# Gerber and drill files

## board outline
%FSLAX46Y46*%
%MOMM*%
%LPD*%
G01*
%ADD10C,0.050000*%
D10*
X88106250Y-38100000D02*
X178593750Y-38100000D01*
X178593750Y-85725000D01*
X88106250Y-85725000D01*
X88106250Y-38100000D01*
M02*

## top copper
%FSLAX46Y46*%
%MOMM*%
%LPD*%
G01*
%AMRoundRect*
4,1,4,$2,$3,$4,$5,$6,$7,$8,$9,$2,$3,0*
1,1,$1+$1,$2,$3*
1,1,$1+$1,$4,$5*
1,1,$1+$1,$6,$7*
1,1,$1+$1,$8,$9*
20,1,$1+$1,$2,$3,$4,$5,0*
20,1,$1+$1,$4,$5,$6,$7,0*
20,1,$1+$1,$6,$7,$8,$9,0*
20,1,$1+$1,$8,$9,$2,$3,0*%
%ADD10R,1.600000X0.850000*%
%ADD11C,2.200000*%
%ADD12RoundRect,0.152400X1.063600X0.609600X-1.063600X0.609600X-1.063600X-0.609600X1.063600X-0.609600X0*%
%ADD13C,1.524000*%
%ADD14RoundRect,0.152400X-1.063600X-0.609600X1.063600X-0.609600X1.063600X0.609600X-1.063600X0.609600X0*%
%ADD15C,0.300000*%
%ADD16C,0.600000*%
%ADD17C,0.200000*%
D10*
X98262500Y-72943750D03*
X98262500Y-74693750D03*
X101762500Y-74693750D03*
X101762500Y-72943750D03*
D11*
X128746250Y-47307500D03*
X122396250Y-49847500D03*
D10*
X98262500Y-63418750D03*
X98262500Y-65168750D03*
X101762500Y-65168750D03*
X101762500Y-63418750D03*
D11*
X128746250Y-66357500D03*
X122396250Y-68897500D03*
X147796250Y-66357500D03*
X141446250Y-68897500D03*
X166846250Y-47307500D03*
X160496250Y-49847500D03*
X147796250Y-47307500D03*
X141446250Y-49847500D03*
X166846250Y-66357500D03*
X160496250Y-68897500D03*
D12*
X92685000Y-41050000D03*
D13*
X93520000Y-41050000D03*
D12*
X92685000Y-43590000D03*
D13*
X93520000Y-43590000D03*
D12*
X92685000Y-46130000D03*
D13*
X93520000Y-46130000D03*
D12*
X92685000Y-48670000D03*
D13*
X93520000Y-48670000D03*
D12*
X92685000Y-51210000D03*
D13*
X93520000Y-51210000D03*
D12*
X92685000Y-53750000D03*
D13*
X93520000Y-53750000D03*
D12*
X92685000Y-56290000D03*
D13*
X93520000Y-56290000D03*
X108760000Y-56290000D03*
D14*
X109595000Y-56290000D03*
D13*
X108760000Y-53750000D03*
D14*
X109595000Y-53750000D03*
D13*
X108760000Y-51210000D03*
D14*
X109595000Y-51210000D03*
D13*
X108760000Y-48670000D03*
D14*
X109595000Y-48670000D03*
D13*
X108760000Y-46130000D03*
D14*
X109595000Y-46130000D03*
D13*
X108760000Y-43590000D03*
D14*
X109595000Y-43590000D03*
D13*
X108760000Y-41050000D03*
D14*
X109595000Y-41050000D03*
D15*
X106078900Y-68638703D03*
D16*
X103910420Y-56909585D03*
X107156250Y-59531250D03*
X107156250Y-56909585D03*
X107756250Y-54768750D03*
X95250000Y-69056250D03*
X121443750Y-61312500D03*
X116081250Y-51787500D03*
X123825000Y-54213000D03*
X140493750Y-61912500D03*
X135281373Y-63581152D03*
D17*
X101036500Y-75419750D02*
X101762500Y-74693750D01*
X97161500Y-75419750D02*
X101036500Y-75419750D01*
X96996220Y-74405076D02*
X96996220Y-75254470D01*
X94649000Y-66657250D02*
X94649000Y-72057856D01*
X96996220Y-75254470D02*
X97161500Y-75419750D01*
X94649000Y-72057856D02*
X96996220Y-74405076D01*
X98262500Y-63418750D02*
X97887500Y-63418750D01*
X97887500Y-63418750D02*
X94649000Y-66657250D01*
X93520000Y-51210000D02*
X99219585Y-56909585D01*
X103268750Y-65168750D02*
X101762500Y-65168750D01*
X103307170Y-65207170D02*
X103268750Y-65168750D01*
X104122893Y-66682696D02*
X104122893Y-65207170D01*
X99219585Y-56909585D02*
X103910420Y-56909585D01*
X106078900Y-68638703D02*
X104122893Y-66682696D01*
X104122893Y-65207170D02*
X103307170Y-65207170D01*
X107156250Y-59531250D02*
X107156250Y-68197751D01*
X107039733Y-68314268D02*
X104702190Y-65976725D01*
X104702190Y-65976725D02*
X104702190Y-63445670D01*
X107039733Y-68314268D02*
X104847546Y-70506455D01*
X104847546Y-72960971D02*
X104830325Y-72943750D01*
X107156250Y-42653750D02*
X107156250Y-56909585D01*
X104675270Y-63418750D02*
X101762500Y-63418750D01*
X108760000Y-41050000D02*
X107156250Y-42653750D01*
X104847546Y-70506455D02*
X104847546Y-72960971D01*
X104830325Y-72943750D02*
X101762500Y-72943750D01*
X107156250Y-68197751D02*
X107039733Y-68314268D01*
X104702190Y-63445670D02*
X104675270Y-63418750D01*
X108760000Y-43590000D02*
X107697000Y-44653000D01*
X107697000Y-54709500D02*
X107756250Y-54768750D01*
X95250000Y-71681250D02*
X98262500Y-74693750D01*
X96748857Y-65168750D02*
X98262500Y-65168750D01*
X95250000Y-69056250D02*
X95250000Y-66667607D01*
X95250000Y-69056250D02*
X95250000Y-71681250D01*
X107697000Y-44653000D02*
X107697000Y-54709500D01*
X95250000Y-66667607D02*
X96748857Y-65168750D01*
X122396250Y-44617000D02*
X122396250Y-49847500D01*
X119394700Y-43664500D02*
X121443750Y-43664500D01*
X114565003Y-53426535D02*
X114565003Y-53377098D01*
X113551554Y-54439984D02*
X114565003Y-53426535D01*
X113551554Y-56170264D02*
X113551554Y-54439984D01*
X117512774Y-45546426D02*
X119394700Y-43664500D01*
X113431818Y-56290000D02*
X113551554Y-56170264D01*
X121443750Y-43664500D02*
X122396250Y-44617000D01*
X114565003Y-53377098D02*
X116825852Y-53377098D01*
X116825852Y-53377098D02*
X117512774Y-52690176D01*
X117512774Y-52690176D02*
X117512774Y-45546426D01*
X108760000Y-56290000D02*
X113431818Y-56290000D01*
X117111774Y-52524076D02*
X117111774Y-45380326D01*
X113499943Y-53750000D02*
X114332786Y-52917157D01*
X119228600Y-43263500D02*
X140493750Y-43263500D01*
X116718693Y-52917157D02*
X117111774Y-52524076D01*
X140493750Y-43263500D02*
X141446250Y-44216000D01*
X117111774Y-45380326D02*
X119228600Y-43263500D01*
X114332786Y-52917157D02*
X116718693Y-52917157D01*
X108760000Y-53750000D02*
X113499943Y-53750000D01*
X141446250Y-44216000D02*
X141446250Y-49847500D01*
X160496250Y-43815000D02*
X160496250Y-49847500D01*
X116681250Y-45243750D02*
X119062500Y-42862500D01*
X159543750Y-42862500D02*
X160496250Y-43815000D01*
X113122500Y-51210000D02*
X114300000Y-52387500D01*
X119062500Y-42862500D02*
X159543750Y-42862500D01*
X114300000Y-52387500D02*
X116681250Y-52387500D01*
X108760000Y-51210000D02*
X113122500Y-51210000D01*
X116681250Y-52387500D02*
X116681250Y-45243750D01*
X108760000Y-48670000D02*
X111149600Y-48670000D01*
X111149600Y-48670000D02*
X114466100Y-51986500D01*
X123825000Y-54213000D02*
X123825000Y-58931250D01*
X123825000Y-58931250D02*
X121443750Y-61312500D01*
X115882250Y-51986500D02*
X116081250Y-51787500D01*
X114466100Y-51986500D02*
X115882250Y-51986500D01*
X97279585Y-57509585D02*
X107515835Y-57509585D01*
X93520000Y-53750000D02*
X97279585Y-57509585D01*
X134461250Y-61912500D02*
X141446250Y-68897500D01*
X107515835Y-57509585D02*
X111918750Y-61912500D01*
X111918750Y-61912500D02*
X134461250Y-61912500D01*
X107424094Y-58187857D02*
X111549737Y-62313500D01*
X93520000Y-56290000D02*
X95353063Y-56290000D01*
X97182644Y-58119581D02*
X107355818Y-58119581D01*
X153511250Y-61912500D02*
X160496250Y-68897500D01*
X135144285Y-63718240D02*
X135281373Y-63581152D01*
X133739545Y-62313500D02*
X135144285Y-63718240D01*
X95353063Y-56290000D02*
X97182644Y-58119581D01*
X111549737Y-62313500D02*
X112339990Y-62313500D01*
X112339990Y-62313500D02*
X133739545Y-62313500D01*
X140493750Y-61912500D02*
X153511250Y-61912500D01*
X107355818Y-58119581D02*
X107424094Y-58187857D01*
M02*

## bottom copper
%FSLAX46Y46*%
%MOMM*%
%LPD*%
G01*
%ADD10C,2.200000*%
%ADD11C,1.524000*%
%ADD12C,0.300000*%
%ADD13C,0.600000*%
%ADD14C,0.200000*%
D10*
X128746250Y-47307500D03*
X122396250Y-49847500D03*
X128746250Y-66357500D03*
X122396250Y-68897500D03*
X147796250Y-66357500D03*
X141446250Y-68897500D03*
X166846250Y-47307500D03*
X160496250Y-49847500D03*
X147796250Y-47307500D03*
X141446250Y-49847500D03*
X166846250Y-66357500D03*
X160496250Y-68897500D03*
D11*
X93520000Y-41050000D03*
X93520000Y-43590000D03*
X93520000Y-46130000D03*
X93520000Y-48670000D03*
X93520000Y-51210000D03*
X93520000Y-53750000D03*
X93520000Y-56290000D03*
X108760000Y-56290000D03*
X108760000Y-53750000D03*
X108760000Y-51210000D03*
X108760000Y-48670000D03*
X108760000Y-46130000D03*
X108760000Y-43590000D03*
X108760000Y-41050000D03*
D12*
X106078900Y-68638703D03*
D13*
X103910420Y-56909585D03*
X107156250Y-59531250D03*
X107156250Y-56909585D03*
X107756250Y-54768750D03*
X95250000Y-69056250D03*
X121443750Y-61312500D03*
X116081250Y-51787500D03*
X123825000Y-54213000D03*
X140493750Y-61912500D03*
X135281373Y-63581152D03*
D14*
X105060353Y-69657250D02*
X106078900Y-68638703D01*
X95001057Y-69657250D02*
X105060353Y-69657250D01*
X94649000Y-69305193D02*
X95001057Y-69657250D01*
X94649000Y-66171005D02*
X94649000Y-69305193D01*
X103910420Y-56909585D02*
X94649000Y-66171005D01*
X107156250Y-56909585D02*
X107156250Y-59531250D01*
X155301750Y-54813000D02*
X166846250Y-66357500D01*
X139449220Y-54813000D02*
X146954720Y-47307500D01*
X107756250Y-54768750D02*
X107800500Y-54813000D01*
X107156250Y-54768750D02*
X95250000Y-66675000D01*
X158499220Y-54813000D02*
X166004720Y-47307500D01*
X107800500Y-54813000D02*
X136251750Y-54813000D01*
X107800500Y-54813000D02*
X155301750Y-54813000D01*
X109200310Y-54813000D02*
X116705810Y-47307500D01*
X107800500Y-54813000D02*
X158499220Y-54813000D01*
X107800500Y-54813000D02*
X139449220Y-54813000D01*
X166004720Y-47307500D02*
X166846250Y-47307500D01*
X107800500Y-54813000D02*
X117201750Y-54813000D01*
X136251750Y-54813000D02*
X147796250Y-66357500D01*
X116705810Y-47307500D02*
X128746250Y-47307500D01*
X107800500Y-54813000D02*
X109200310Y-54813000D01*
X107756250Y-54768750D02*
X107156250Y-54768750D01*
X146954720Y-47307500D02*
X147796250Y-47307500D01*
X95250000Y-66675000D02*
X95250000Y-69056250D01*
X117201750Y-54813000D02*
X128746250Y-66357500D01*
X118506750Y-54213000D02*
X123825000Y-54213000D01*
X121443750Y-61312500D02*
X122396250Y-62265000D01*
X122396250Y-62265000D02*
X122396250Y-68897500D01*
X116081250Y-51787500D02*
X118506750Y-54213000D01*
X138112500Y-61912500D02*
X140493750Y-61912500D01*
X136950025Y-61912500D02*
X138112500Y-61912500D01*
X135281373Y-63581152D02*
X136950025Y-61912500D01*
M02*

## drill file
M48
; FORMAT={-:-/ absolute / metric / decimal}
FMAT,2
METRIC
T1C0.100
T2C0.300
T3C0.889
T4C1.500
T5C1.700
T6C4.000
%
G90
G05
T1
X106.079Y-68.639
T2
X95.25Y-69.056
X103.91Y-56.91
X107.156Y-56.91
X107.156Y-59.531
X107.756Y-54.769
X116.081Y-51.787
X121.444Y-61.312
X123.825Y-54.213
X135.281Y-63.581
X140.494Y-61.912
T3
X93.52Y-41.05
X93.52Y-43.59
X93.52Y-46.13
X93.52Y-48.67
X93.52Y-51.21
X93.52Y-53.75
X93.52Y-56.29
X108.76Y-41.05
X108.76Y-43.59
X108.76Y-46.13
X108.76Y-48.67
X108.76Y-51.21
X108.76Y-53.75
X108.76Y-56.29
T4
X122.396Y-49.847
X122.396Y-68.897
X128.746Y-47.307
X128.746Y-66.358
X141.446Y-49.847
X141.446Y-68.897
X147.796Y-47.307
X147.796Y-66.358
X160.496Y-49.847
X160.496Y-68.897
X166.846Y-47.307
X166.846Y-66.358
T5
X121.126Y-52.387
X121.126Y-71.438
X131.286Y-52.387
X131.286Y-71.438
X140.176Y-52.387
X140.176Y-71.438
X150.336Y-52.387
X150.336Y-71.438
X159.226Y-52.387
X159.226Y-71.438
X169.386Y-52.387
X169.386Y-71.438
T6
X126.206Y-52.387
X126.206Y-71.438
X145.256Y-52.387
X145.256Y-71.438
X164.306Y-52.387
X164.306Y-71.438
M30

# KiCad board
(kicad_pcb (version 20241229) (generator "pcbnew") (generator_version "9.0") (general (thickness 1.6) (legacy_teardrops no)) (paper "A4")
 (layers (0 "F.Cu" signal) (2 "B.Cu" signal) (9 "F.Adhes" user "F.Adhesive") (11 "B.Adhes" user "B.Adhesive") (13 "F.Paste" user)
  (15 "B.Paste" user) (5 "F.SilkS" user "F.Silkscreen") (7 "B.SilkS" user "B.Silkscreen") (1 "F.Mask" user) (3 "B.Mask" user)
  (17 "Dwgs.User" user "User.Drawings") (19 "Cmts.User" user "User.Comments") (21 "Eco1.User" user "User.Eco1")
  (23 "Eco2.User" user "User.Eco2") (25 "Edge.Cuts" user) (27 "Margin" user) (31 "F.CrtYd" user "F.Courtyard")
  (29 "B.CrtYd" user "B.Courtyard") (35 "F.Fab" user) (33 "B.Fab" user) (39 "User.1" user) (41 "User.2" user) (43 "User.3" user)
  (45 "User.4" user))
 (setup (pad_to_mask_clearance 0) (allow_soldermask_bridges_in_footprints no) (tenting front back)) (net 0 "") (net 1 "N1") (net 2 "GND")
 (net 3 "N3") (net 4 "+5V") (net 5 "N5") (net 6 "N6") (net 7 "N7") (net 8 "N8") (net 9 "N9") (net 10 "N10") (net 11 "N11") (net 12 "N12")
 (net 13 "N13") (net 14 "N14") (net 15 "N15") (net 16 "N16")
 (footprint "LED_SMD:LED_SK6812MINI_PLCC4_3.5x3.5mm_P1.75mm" (layer "F.Cu") (at 100.0125 73.81875)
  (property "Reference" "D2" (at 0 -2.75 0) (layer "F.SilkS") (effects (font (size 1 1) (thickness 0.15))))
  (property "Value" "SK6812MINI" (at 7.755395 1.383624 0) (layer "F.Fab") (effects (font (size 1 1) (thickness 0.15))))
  (pad "1" smd rect (at -1.75 -0.875) (size 1.6 0.85) (layers "F.Cu" "F.Mask" "F.Paste") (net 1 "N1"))
  (pad "2" smd rect (at -1.75 0.875) (size 1.6 0.85) (layers "F.Cu" "F.Mask" "F.Paste") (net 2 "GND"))
  (pad "3" smd rect (at 1.75 0.875) (size 1.6 0.85) (layers "F.Cu" "F.Mask" "F.Paste") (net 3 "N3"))
  (pad "4" smd rect (at 1.75 -0.875) (size 1.6 0.85) (layers "F.Cu" "F.Mask" "F.Paste") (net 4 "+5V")))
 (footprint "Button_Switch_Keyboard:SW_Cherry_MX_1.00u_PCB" (layer "F.Cu") (at 128.74625 47.3075)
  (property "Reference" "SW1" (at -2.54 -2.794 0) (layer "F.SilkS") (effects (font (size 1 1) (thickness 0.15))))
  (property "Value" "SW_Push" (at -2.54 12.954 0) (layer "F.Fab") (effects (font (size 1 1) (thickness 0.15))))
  (pad "" np_thru_hole circle (at -7.62 5.08) (size 1.7 1.7) (drill 1.7) (layers "*.Cu" "*.Mask"))
  (pad "" np_thru_hole circle (at -2.54 5.08) (size 4 4) (drill 4) (layers "*.Cu" "*.Mask"))
  (pad "" np_thru_hole circle (at 2.54 5.08) (size 1.7 1.7) (drill 1.7) (layers "*.Cu" "*.Mask"))
  (pad "1" thru_hole circle (at 0 0) (size 2.2 2.2) (drill 1.5) (layers "*.Cu" "*.Mask") (remove_unused_layers no) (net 2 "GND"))
  (pad "2" thru_hole circle (at -6.35 2.54) (size 2.2 2.2) (drill 1.5) (layers "*.Cu" "*.Mask") (remove_unused_layers no) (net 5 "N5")))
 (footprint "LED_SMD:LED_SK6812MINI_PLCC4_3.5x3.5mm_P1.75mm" (layer "F.Cu") (at 100.0125 64.29375)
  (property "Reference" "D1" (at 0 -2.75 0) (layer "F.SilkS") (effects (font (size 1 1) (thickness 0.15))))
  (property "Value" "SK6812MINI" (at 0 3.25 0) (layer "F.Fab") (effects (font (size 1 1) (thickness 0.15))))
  (pad "1" smd rect (at -1.75 -0.875) (size 1.6 0.85) (layers "F.Cu" "F.Mask" "F.Paste") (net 3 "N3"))
  (pad "2" smd rect (at -1.75 0.875) (size 1.6 0.85) (layers "F.Cu" "F.Mask" "F.Paste") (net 2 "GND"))
  (pad "3" smd rect (at 1.75 0.875) (size 1.6 0.85) (layers "F.Cu" "F.Mask" "F.Paste") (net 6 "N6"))
  (pad "4" smd rect (at 1.75 -0.875) (size 1.6 0.85) (layers "F.Cu" "F.Mask" "F.Paste") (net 4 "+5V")))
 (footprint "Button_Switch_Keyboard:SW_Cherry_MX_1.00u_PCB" (layer "F.Cu") (at 128.74625 66.3575)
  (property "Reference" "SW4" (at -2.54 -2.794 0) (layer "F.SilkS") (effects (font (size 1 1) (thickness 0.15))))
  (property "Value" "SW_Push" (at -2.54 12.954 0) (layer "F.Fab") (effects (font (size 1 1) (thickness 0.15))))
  (pad "" np_thru_hole circle (at -7.62 5.08) (size 1.7 1.7) (drill 1.7) (layers "*.Cu" "*.Mask"))
  (pad "" np_thru_hole circle (at -2.54 5.08) (size 4 4) (drill 4) (layers "*.Cu" "*.Mask"))
  (pad "" np_thru_hole circle (at 2.54 5.08) (size 1.7 1.7) (drill 1.7) (layers "*.Cu" "*.Mask"))
  (pad "1" thru_hole circle (at 0 0) (size 2.2 2.2) (drill 1.5) (layers "*.Cu" "*.Mask") (remove_unused_layers no) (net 2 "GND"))
  (pad "2" thru_hole circle (at -6.35 2.54) (size 2.2 2.2) (drill 1.5) (layers "*.Cu" "*.Mask") (remove_unused_layers no) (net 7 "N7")))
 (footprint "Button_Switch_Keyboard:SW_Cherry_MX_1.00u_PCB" (layer "F.Cu") (at 147.79625 66.3575)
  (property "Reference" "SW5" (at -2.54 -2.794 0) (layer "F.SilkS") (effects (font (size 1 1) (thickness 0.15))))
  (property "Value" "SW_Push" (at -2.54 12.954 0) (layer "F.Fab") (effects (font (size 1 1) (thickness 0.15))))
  (pad "" np_thru_hole circle (at -7.62 5.08) (size 1.7 1.7) (drill 1.7) (layers "*.Cu" "*.Mask"))
  (pad "" np_thru_hole circle (at -2.54 5.08) (size 4 4) (drill 4) (layers "*.Cu" "*.Mask"))
  (pad "" np_thru_hole circle (at 2.54 5.08) (size 1.7 1.7) (drill 1.7) (layers "*.Cu" "*.Mask"))
  (pad "1" thru_hole circle (at 0 0) (size 2.2 2.2) (drill 1.5) (layers "*.Cu" "*.Mask") (remove_unused_layers no) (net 2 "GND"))
  (pad "2" thru_hole circle (at -6.35 2.54) (size 2.2 2.2) (drill 1.5) (layers "*.Cu" "*.Mask") (remove_unused_layers no) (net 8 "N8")))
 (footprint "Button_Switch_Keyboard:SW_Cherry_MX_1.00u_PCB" (layer "F.Cu") (at 166.84625 47.3075)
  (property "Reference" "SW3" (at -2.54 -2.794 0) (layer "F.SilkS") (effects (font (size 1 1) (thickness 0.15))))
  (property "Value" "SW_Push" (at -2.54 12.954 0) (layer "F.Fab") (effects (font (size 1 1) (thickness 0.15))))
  (pad "" np_thru_hole circle (at -7.62 5.08) (size 1.7 1.7) (drill 1.7) (layers "*.Cu" "*.Mask"))
  (pad "" np_thru_hole circle (at -2.54 5.08) (size 4 4) (drill 4) (layers "*.Cu" "*.Mask"))
  (pad "" np_thru_hole circle (at 2.54 5.08) (size 1.7 1.7) (drill 1.7) (layers "*.Cu" "*.Mask"))
  (pad "1" thru_hole circle (at 0 0) (size 2.2 2.2) (drill 1.5) (layers "*.Cu" "*.Mask") (remove_unused_layers no) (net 2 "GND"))
  (pad "2" thru_hole circle (at -6.35 2.54) (size 2.2 2.2) (drill 1.5) (layers "*.Cu" "*.Mask") (remove_unused_layers no) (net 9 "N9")))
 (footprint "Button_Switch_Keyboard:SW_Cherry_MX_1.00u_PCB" (layer "F.Cu") (at 147.79625 47.3075)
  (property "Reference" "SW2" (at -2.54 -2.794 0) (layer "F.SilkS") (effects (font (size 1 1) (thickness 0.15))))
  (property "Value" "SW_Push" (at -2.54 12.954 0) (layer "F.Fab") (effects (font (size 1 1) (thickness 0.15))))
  (pad "" np_thru_hole circle (at -7.62 5.08) (size 1.7 1.7) (drill 1.7) (layers "*.Cu" "*.Mask"))
  (pad "" np_thru_hole circle (at -2.54 5.08) (size 4 4) (drill 4) (layers "*.Cu" "*.Mask"))
  (pad "" np_thru_hole circle (at 2.54 5.08) (size 1.7 1.7) (drill 1.7) (layers "*.Cu" "*.Mask"))
  (pad "1" thru_hole circle (at 0 0) (size 2.2 2.2) (drill 1.5) (layers "*.Cu" "*.Mask") (remove_unused_layers no) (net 2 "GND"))
  (pad "2" thru_hole circle (at -6.35 2.54) (size 2.2 2.2) (drill 1.5) (layers "*.Cu" "*.Mask") (remove_unused_layers no) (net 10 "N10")))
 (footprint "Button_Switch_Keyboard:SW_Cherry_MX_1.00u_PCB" (layer "F.Cu") (at 166.84625 66.3575)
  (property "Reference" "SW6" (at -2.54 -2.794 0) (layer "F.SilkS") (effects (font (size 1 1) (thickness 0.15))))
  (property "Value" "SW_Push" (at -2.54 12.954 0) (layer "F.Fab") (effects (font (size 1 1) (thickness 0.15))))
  (pad "" np_thru_hole circle (at -7.62 5.08) (size 1.7 1.7) (drill 1.7) (layers "*.Cu" "*.Mask"))
  (pad "" np_thru_hole circle (at -2.54 5.08) (size 4 4) (drill 4) (layers "*.Cu" "*.Mask"))
  (pad "" np_thru_hole circle (at 2.54 5.08) (size 1.7 1.7) (drill 1.7) (layers "*.Cu" "*.Mask"))
  (pad "1" thru_hole circle (at 0 0) (size 2.2 2.2) (drill 1.5) (layers "*.Cu" "*.Mask") (remove_unused_layers no) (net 2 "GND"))
  (pad "2" thru_hole circle (at -6.35 2.54) (size 2.2 2.2) (drill 1.5) (layers "*.Cu" "*.Mask") (remove_unused_layers no) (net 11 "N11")))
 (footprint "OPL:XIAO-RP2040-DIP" (layer "F.Cu") (at 101.14 48.67)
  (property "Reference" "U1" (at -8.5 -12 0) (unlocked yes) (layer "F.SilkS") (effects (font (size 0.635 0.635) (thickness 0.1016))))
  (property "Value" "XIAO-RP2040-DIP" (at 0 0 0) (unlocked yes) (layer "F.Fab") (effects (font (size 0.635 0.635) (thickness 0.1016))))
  (pad "1" smd roundrect (at -8.455 -7.62 180) (size 2.432 1.524) (layers "F.Cu" "F.Mask") (roundrect_rratio 0.1) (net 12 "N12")
   (thermal_bridge_angle 45))
  (pad "1" thru_hole circle (at -7.62 -7.62 180) (size 1.524 1.524) (drill 0.889) (layers "*.Cu" "*.Mask") (remove_unused_layers no)
   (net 12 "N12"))
  (pad "2" smd roundrect (at -8.455 -5.08 180) (size 2.432 1.524) (layers "F.Cu" "F.Mask") (roundrect_rratio 0.1) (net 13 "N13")
   (thermal_bridge_angle 45))
  (pad "2" thru_hole circle (at -7.62 -5.08 180) (size 1.524 1.524) (drill 0.889) (layers "*.Cu" "*.Mask") (remove_unused_layers no)
   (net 13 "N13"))
  (pad "3" smd roundrect (at -8.455 -2.54 180) (size 2.432 1.524) (layers "F.Cu" "F.Mask") (roundrect_rratio 0.1) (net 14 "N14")
   (thermal_bridge_angle 45))
  (pad "3" thru_hole circle (at -7.62 -2.54 180) (size 1.524 1.524) (drill 0.889) (layers "*.Cu" "*.Mask") (remove_unused_layers no)
   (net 14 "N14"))
  (pad "4" smd roundrect (at -8.455 0 180) (size 2.432 1.524) (layers "F.Cu" "F.Mask") (roundrect_rratio 0.1) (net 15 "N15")
   (thermal_bridge_angle 45))
  (pad "4" thru_hole circle (at -7.62 0 180) (size 1.524 1.524) (drill 0.889) (layers "*.Cu" "*.Mask") (remove_unused_layers no)
   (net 15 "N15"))
  (pad "5" smd roundrect (at -8.455 2.54 180) (size 2.432 1.524) (layers "F.Cu" "F.Mask") (roundrect_rratio 0.1) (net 6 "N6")
   (thermal_bridge_angle 45))
  (pad "5" thru_hole circle (at -7.62 2.54 180) (size 1.524 1.524) (drill 0.889) (layers "*.Cu" "*.Mask") (remove_unused_layers no)
   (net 6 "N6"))
  (pad "6" smd roundrect (at -8.455 5.08 180) (size 2.432 1.524) (layers "F.Cu" "F.Mask") (roundrect_rratio 0.1) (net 8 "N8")
   (thermal_bridge_angle 45))
  (pad "6" thru_hole circle (at -7.62 5.08 180) (size 1.524 1.524) (drill 0.889) (layers "*.Cu" "*.Mask") (remove_unused_layers no)
   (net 8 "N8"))
  (pad "7" smd roundrect (at -8.455 7.62 180) (size 2.432 1.524) (layers "F.Cu" "F.Mask") (roundrect_rratio 0.1) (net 11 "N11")
   (thermal_bridge_angle 45))
  (pad "7" thru_hole circle (at -7.62 7.62 180) (size 1.524 1.524) (drill 0.889) (layers "*.Cu" "*.Mask") (remove_unused_layers no)
   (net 11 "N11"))
  (pad "8" thru_hole circle (at 7.62 7.62) (size 1.524 1.524) (drill 0.889) (layers "*.Cu" "*.Mask") (remove_unused_layers no) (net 5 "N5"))
  (pad "8" smd roundrect (at 8.455 7.62) (size 2.432 1.524) (layers "F.Cu" "F.Mask") (roundrect_rratio 0.1) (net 5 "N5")
   (thermal_bridge_angle 45))
  (pad "9" thru_hole circle (at 7.62 5.08) (size 1.524 1.524) (drill 0.889) (layers "*.Cu" "*.Mask") (remove_unused_layers no)
   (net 10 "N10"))
  (pad "9" smd roundrect (at 8.455 5.08) (size 2.432 1.524) (layers "F.Cu" "F.Mask") (roundrect_rratio 0.1) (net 10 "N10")
   (thermal_bridge_angle 45))
  (pad "10" thru_hole circle (at 7.62 2.54) (size 1.524 1.524) (drill 0.889) (layers "*.Cu" "*.Mask") (remove_unused_layers no) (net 9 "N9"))
  (pad "10" smd roundrect (at 8.455 2.54) (size 2.432 1.524) (layers "F.Cu" "F.Mask") (roundrect_rratio 0.1) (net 9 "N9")
   (thermal_bridge_angle 45))
  (pad "11" thru_hole circle (at 7.62 0) (size 1.524 1.524) (drill 0.889) (layers "*.Cu" "*.Mask") (remove_unused_layers no) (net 7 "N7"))
  (pad "11" smd roundrect (at 8.455 0) (size 2.432 1.524) (layers "F.Cu" "F.Mask") (roundrect_rratio 0.1) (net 7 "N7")
   (thermal_bridge_angle 45))
  (pad "12" thru_hole circle (at 7.62 -2.54) (size 1.524 1.524) (drill 0.889) (layers "*.Cu" "*.Mask") (remove_unused_layers no)
   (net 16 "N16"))
  (pad "12" smd roundrect (at 8.455 -2.54) (size 2.432 1.524) (layers "F.Cu" "F.Mask") (roundrect_rratio 0.1) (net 16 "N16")
   (thermal_bridge_angle 45))
  (pad "13" thru_hole circle (at 7.62 -5.08) (size 1.524 1.524) (drill 0.889) (layers "*.Cu" "*.Mask") (remove_unused_layers no)
   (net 2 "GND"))
  (pad "13" smd roundrect (at 8.455 -5.08) (size 2.432 1.524) (layers "F.Cu" "F.Mask") (roundrect_rratio 0.1) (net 2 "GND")
   (thermal_bridge_angle 45))
  (pad "14" thru_hole circle (at 7.62 -7.62) (size 1.524 1.524) (drill 0.889) (layers "*.Cu" "*.Mask") (remove_unused_layers no)
   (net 4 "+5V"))
  (pad "14" smd roundrect (at 8.455 -7.62) (size 2.432 1.524) (layers "F.Cu" "F.Mask") (roundrect_rratio 0.1) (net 4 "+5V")
   (thermal_bridge_angle 45)))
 (gr_rect (start 88.10625 38.1) (end 178.59375 85.725) (stroke (width 0.05) (type default)) (fill no) (layer "Edge.Cuts"))
 (segment (start 101.0365 75.41975) (end 101.7625 74.69375) (width 0.2) (layer "F.Cu") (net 3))
 (segment (start 97.1615 75.41975) (end 101.0365 75.41975) (width 0.2) (layer "F.Cu") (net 3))
 (segment (start 96.99622 74.405076) (end 96.99622 75.25447) (width 0.2) (layer "F.Cu") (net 3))
 (segment (start 94.649 66.65725) (end 94.649 72.057856) (width 0.2) (layer "F.Cu") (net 3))
 (segment (start 96.99622 75.25447) (end 97.1615 75.41975) (width 0.2) (layer "F.Cu") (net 3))
 (segment (start 94.649 72.057856) (end 96.99622 74.405076) (width 0.2) (layer "F.Cu") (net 3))
 (segment (start 98.2625 63.41875) (end 97.8875 63.41875) (width 0.2) (layer "F.Cu") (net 3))
 (segment (start 97.8875 63.41875) (end 94.649 66.65725) (width 0.2) (layer "F.Cu") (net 3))
 (segment (start 93.52 51.21) (end 99.219585 56.909585) (width 0.2) (layer "F.Cu") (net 6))
 (segment (start 103.26875 65.16875) (end 101.7625 65.16875) (width 0.2) (layer "F.Cu") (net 6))
 (segment (start 103.30717 65.20717) (end 103.26875 65.16875) (width 0.2) (layer "F.Cu") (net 6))
 (segment (start 104.122893 66.682696) (end 104.122893 65.20717) (width 0.2) (layer "F.Cu") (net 6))
 (segment (start 99.219585 56.909585) (end 103.91042 56.909585) (width 0.2) (layer "F.Cu") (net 6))
 (segment (start 106.0789 68.638703) (end 104.122893 66.682696) (width 0.2) (layer "F.Cu") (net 6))
 (segment (start 104.122893 65.20717) (end 103.30717 65.20717) (width 0.2) (layer "F.Cu") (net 6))
 (via micro (at 106.0789 68.638703) (size 0.3) (drill 0.1) (layers "F.Cu" "B.Cu") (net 6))
 (via (at 103.91042 56.909585) (size 0.6) (drill 0.3) (layers "F.Cu" "B.Cu") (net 6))
 (segment (start 105.060353 69.65725) (end 106.0789 68.638703) (width 0.2) (layer "B.Cu") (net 6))
 (segment (start 95.001057 69.65725) (end 105.060353 69.65725) (width 0.2) (layer "B.Cu") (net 6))
 (segment (start 94.649 69.305193) (end 95.001057 69.65725) (width 0.2) (layer "B.Cu") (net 6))
 (segment (start 94.649 66.171005) (end 94.649 69.305193) (width 0.2) (layer "B.Cu") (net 6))
 (segment (start 103.91042 56.909585) (end 94.649 66.171005) (width 0.2) (layer "B.Cu") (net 6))
 (segment (start 107.15625 59.53125) (end 107.15625 68.197751) (width 0.2) (layer "F.Cu") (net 4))
 (segment (start 107.039733 68.314268) (end 104.70219 65.976725) (width 0.2) (layer "F.Cu") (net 4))
 (segment (start 104.70219 65.976725) (end 104.70219 63.44567) (width 0.2) (layer "F.Cu") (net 4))
 (segment (start 107.039733 68.314268) (end 104.847546 70.506455) (width 0.2) (layer "F.Cu") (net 4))
 (segment (start 104.847546 72.960971) (end 104.830325 72.94375) (width 0.2) (layer "F.Cu") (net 4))
 (segment (start 107.15625 42.65375) (end 107.15625 56.909585) (width 0.2) (layer "F.Cu") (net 4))
 (segment (start 104.67527 63.41875) (end 101.7625 63.41875) (width 0.2) (layer "F.Cu") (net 4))
 (segment (start 108.76 41.05) (end 107.15625 42.65375) (width 0.2) (layer "F.Cu") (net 4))
 (segment (start 104.847546 70.506455) (end 104.847546 72.960971) (width 0.2) (layer "F.Cu") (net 4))
 (segment (start 104.830325 72.94375) (end 101.7625 72.94375) (width 0.2) (layer "F.Cu") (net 4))
 (segment (start 107.15625 68.197751) (end 107.039733 68.314268) (width 0.2) (layer "F.Cu") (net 4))
 (segment (start 104.70219 63.44567) (end 104.67527 63.41875) (width 0.2) (layer "F.Cu") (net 4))
 (via (at 107.15625 59.53125) (size 0.6) (drill 0.3) (layers "F.Cu" "B.Cu") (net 4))
 (via (at 107.15625 56.909585) (size 0.6) (drill 0.3) (layers "F.Cu" "B.Cu") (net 4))
 (segment (start 107.15625 56.909585) (end 107.15625 59.53125) (width 0.2) (layer "B.Cu") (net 4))
 (segment (start 108.76 43.59) (end 107.697 44.653) (width 0.2) (layer "F.Cu") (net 2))
 (segment (start 107.697 54.7095) (end 107.75625 54.76875) (width 0.2) (layer "F.Cu") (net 2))
 (segment (start 95.25 71.68125) (end 98.2625 74.69375) (width 0.2) (layer "F.Cu") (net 2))
 (segment (start 96.748857 65.16875) (end 98.2625 65.16875) (width 0.2) (layer "F.Cu") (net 2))
 (segment (start 95.25 69.05625) (end 95.25 66.667607) (width 0.2) (layer "F.Cu") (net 2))
 (segment (start 95.25 69.05625) (end 95.25 71.68125) (width 0.2) (layer "F.Cu") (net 2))
 (segment (start 107.697 44.653) (end 107.697 54.7095) (width 0.2) (layer "F.Cu") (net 2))
 (segment (start 95.25 66.667607) (end 96.748857 65.16875) (width 0.2) (layer "F.Cu") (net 2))
 (via (at 107.75625 54.76875) (size 0.6) (drill 0.3) (layers "F.Cu" "B.Cu") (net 2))
 (via (at 95.25 69.05625) (size 0.6) (drill 0.3) (layers "F.Cu" "B.Cu") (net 2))
 (segment (start 155.30175 54.813) (end 166.84625 66.3575) (width 0.2) (layer "B.Cu") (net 2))
 (segment (start 139.44922 54.813) (end 146.95472 47.3075) (width 0.2) (layer "B.Cu") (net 2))
 (segment (start 107.75625 54.76875) (end 107.8005 54.813) (width 0.2) (layer "B.Cu") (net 2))
 (segment (start 107.15625 54.76875) (end 95.25 66.675) (width 0.2) (layer "B.Cu") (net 2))
 (segment (start 158.49922 54.813) (end 166.00472 47.3075) (width 0.2) (layer "B.Cu") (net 2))
 (segment (start 107.8005 54.813) (end 136.25175 54.813) (width 0.2) (layer "B.Cu") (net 2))
 (segment (start 107.8005 54.813) (end 155.30175 54.813) (width 0.2) (layer "B.Cu") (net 2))
 (segment (start 109.20031 54.813) (end 116.70581 47.3075) (width 0.2) (layer "B.Cu") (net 2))
 (segment (start 107.8005 54.813) (end 158.49922 54.813) (width 0.2) (layer "B.Cu") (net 2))
 (segment (start 107.8005 54.813) (end 139.44922 54.813) (width 0.2) (layer "B.Cu") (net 2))
 (segment (start 166.00472 47.3075) (end 166.84625 47.3075) (width 0.2) (layer "B.Cu") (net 2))
 (segment (start 107.8005 54.813) (end 117.20175 54.813) (width 0.2) (layer "B.Cu") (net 2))
 (segment (start 136.25175 54.813) (end 147.79625 66.3575) (width 0.2) (layer "B.Cu") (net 2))
 (segment (start 116.70581 47.3075) (end 128.74625 47.3075) (width 0.2) (layer "B.Cu") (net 2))
 (segment (start 107.8005 54.813) (end 109.20031 54.813) (width 0.2) (layer "B.Cu") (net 2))
 (segment (start 107.75625 54.76875) (end 107.15625 54.76875) (width 0.2) (layer "B.Cu") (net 2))
 (segment (start 146.95472 47.3075) (end 147.79625 47.3075) (width 0.2) (layer "B.Cu") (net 2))
 (segment (start 95.25 66.675) (end 95.25 69.05625) (width 0.2) (layer "B.Cu") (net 2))
 (segment (start 117.20175 54.813) (end 128.74625 66.3575) (width 0.2) (layer "B.Cu") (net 2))
 (segment (start 122.39625 44.617) (end 122.39625 49.8475) (width 0.2) (layer "F.Cu") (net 5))
 (segment (start 119.3947 43.6645) (end 121.44375 43.6645) (width 0.2) (layer "F.Cu") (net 5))
 (segment (start 114.565003 53.426535) (end 114.565003 53.377098) (width 0.2) (layer "F.Cu") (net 5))
 (segment (start 113.551554 54.439984) (end 114.565003 53.426535) (width 0.2) (layer "F.Cu") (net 5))
 (segment (start 113.551554 56.170264) (end 113.551554 54.439984) (width 0.2) (layer "F.Cu") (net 5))
 (segment (start 117.512774 45.546426) (end 119.3947 43.6645) (width 0.2) (layer "F.Cu") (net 5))
 (segment (start 113.431818 56.29) (end 113.551554 56.170264) (width 0.2) (layer "F.Cu") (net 5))
 (segment (start 121.44375 43.6645) (end 122.39625 44.617) (width 0.2) (layer "F.Cu") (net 5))
 (segment (start 114.565003 53.377098) (end 116.825852 53.377098) (width 0.2) (layer "F.Cu") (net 5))
 (segment (start 116.825852 53.377098) (end 117.512774 52.690176) (width 0.2) (layer "F.Cu") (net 5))
 (segment (start 117.512774 52.690176) (end 117.512774 45.546426) (width 0.2) (layer "F.Cu") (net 5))
 (segment (start 108.76 56.29) (end 113.431818 56.29) (width 0.2) (layer "F.Cu") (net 5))
 (segment (start 117.111774 52.524076) (end 117.111774 45.380326) (width 0.2) (layer "F.Cu") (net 10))
 (segment (start 113.499943 53.75) (end 114.332786 52.917157) (width 0.2) (layer "F.Cu") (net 10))
 (segment (start 119.2286 43.2635) (end 140.49375 43.2635) (width 0.2) (layer "F.Cu") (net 10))
 (segment (start 116.718693 52.917157) (end 117.111774 52.524076) (width 0.2) (layer "F.Cu") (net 10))
 (segment (start 140.49375 43.2635) (end 141.44625 44.216) (width 0.2) (layer "F.Cu") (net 10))
 (segment (start 117.111774 45.380326) (end 119.2286 43.2635) (width 0.2) (layer "F.Cu") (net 10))
 (segment (start 114.332786 52.917157) (end 116.718693 52.917157) (width 0.2) (layer "F.Cu") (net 10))
 (segment (start 108.76 53.75) (end 113.499943 53.75) (width 0.2) (layer "F.Cu") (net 10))
 (segment (start 141.44625 44.216) (end 141.44625 49.8475) (width 0.2) (layer "F.Cu") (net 10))
 (segment (start 160.49625 43.815) (end 160.49625 49.8475) (width 0.2) (layer "F.Cu") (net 9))
 (segment (start 116.68125 45.24375) (end 119.0625 42.8625) (width 0.2) (layer "F.Cu") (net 9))
 (segment (start 159.54375 42.8625) (end 160.49625 43.815) (width 0.2) (layer "F.Cu") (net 9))
 (segment (start 113.1225 51.21) (end 114.3 52.3875) (width 0.2) (layer "F.Cu") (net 9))
 (segment (start 119.0625 42.8625) (end 159.54375 42.8625) (width 0.2) (layer "F.Cu") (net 9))
 (segment (start 114.3 52.3875) (end 116.68125 52.3875) (width 0.2) (layer "F.Cu") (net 9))
 (segment (start 108.76 51.21) (end 113.1225 51.21) (width 0.2) (layer "F.Cu") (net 9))
 (segment (start 116.68125 52.3875) (end 116.68125 45.24375) (width 0.2) (layer "F.Cu") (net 9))
 (segment (start 108.76 48.67) (end 111.1496 48.67) (width 0.2) (layer "F.Cu") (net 7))
 (segment (start 111.1496 48.67) (end 114.4661 51.9865) (width 0.2) (layer "F.Cu") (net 7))
 (segment (start 123.825 54.213) (end 123.825 58.93125) (width 0.2) (layer "F.Cu") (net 7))
 (segment (start 123.825 58.93125) (end 121.44375 61.3125) (width 0.2) (layer "F.Cu") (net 7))
 (segment (start 115.88225 51.9865) (end 116.08125 51.7875) (width 0.2) (layer "F.Cu") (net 7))
 (segment (start 114.4661 51.9865) (end 115.88225 51.9865) (width 0.2) (layer "F.Cu") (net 7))
 (via (at 121.44375 61.3125) (size 0.6) (drill 0.3) (layers "F.Cu" "B.Cu") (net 7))
 (via (at 116.08125 51.7875) (size 0.6) (drill 0.3) (layers "F.Cu" "B.Cu") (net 7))
 (via (at 123.825 54.213) (size 0.6) (drill 0.3) (layers "F.Cu" "B.Cu") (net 7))
 (segment (start 118.50675 54.213) (end 123.825 54.213) (width 0.2) (layer "B.Cu") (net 7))
 (segment (start 121.44375 61.3125) (end 122.39625 62.265) (width 0.2) (layer "B.Cu") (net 7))
 (segment (start 122.39625 62.265) (end 122.39625 68.8975) (width 0.2) (layer "B.Cu") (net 7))
 (segment (start 116.08125 51.7875) (end 118.50675 54.213) (width 0.2) (layer "B.Cu") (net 7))
 (segment (start 97.279585 57.509585) (end 107.515835 57.509585) (width 0.2) (layer "F.Cu") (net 8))
 (segment (start 93.52 53.75) (end 97.279585 57.509585) (width 0.2) (layer "F.Cu") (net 8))
 (segment (start 134.46125 61.9125) (end 141.44625 68.8975) (width 0.2) (layer "F.Cu") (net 8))
 (segment (start 107.515835 57.509585) (end 111.91875 61.9125) (width 0.2) (layer "F.Cu") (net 8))
 (segment (start 111.91875 61.9125) (end 134.46125 61.9125) (width 0.2) (layer "F.Cu") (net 8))
 (segment (start 107.424094 58.187857) (end 111.549737 62.3135) (width 0.2) (layer "F.Cu") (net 11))
 (segment (start 93.52 56.29) (end 95.353063 56.29) (width 0.2) (layer "F.Cu") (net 11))
 (segment (start 97.182644 58.119581) (end 107.355818 58.119581) (width 0.2) (layer "F.Cu") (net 11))
 (segment (start 153.51125 61.9125) (end 160.49625 68.8975) (width 0.2) (layer "F.Cu") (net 11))
 (segment (start 135.144285 63.71824) (end 135.281373 63.581152) (width 0.2) (layer "F.Cu") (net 11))
 (segment (start 133.739545 62.3135) (end 135.144285 63.71824) (width 0.2) (layer "F.Cu") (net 11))
 (segment (start 95.353063 56.29) (end 97.182644 58.119581) (width 0.2) (layer "F.Cu") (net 11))
 (segment (start 111.549737 62.3135) (end 112.33999 62.3135) (width 0.2) (layer "F.Cu") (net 11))
 (segment (start 112.33999 62.3135) (end 133.739545 62.3135) (width 0.2) (layer "F.Cu") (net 11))
 (segment (start 140.49375 61.9125) (end 153.51125 61.9125) (width 0.2) (layer "F.Cu") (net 11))
 (segment (start 107.355818 58.119581) (end 107.424094 58.187857) (width 0.2) (layer "F.Cu") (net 11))
 (via (at 140.49375 61.9125) (size 0.6) (drill 0.3) (layers "F.Cu" "B.Cu") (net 11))
 (via (at 135.281373 63.581152) (size 0.6) (drill 0.3) (layers "F.Cu" "B.Cu") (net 11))
 (segment (start 138.1125 61.9125) (end 140.49375 61.9125) (width 0.2) (layer "B.Cu") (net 11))
 (segment (start 136.950025 61.9125) (end 138.1125 61.9125) (width 0.2) (layer "B.Cu") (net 11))
 (segment (start 135.281373 63.581152) (end 136.950025 61.9125) (width 0.2) (layer "B.Cu") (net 11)))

